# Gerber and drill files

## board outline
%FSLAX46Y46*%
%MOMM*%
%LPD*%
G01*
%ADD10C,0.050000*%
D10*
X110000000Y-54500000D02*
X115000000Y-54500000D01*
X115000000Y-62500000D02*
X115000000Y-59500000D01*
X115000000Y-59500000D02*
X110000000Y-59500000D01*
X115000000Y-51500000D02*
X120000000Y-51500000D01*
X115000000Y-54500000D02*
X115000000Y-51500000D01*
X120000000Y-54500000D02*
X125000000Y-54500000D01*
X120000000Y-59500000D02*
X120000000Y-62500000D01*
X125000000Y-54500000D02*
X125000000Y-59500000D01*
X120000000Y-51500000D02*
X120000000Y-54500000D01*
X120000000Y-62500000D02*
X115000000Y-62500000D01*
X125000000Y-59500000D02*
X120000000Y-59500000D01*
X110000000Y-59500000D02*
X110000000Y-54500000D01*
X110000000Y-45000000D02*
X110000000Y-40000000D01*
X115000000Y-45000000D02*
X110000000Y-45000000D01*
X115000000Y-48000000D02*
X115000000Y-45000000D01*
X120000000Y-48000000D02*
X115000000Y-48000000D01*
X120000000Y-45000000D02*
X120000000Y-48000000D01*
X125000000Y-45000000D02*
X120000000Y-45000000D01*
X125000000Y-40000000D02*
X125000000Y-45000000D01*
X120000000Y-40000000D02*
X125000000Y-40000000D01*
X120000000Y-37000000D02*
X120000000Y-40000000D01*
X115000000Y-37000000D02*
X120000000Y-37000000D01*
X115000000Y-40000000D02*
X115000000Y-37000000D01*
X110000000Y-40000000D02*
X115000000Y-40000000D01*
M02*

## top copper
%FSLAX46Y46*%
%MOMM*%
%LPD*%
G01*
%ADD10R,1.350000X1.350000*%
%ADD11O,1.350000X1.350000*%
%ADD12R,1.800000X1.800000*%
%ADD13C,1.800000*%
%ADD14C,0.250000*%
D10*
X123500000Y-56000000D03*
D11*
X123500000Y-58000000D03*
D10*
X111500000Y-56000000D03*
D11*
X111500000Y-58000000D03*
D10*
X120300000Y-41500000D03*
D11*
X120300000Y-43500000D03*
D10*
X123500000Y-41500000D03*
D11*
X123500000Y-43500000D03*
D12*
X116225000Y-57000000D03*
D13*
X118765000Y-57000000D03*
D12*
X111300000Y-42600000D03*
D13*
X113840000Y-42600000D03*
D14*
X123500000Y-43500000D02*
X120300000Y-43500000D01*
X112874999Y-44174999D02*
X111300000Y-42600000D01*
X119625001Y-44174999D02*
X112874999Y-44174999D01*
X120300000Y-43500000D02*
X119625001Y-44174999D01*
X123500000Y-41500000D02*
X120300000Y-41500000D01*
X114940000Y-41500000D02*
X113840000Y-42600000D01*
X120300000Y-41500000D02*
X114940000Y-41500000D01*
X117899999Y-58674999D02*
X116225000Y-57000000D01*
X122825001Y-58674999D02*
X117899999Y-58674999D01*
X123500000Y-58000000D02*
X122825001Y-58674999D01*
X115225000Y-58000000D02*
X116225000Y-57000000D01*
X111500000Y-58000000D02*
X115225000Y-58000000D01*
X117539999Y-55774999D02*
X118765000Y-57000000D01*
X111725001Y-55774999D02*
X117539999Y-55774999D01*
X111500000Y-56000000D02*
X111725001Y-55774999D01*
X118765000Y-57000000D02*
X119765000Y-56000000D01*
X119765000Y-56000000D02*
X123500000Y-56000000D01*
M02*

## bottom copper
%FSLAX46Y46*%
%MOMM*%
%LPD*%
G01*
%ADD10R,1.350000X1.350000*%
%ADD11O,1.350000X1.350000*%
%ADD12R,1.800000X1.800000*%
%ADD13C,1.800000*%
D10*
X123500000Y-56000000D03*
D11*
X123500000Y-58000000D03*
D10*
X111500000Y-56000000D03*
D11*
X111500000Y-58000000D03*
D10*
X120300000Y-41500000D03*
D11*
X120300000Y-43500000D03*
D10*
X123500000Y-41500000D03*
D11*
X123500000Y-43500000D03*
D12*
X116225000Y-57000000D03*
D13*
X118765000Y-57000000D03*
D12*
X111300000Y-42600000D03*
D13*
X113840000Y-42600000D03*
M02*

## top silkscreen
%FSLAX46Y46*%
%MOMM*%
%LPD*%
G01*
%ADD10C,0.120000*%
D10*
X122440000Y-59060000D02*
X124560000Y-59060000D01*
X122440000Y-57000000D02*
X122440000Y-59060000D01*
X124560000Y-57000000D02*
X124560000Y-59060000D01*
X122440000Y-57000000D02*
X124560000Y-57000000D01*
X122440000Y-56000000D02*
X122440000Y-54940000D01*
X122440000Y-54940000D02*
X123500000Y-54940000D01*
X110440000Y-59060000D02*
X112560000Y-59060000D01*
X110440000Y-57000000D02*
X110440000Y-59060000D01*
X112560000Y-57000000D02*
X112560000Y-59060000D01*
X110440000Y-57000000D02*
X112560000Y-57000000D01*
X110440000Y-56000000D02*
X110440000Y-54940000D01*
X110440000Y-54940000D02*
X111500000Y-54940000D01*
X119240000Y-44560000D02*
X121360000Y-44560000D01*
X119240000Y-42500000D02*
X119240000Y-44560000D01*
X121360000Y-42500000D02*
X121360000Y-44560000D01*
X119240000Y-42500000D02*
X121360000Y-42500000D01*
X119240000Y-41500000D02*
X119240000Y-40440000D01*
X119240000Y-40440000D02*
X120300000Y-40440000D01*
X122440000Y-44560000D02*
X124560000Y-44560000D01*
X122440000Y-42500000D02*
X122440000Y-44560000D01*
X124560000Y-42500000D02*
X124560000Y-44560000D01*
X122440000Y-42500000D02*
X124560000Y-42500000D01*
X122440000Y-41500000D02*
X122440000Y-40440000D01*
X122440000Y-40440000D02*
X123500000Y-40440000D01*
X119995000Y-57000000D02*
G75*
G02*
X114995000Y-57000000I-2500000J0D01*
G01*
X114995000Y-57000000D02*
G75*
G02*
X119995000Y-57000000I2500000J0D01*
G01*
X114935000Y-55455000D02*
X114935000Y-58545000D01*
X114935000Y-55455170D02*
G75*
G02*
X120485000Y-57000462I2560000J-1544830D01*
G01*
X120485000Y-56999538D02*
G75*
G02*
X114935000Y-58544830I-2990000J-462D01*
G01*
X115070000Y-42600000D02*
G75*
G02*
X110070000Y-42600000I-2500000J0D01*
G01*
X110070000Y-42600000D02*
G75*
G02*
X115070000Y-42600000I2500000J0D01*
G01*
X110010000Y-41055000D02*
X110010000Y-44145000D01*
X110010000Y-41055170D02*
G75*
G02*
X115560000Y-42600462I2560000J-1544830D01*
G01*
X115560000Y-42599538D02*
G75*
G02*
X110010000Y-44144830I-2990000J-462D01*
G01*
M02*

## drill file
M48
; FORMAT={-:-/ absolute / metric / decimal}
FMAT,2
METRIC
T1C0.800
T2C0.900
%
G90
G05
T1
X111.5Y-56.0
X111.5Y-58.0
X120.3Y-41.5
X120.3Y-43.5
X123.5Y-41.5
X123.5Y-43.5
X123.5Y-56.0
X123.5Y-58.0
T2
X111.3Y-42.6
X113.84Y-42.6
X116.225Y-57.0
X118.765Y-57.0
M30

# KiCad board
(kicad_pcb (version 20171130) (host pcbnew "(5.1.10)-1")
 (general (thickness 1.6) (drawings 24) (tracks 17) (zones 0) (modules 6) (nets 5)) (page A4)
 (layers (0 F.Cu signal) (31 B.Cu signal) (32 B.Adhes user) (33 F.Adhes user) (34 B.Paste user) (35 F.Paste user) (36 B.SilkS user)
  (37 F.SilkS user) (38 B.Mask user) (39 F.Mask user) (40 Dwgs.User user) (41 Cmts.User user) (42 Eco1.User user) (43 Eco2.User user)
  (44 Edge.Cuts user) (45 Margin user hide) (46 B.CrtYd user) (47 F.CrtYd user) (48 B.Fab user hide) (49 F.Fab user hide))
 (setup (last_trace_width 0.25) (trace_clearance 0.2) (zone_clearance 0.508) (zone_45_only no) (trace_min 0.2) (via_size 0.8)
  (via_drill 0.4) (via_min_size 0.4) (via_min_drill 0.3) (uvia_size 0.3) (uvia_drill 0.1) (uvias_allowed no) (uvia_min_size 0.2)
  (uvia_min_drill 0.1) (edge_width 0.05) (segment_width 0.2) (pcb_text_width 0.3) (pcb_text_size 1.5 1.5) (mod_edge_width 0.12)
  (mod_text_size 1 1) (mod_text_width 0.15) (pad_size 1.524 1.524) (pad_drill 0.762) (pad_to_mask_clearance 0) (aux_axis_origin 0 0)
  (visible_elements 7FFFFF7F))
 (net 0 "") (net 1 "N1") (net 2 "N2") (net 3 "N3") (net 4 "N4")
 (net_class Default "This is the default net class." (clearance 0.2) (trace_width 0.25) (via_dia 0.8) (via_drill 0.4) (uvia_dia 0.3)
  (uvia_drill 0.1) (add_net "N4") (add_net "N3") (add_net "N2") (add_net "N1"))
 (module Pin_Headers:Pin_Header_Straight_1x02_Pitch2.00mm (layer F.Cu) (at 123.5 56)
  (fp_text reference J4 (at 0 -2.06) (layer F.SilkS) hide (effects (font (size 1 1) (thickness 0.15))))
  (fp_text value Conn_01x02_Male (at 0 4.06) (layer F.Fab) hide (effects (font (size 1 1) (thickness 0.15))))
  (fp_line (start -1.06 3.06) (end 1.06 3.06) (layer F.SilkS) (width 0.12))
  (fp_line (start -1.06 1) (end -1.06 3.06) (layer F.SilkS) (width 0.12))
  (fp_line (start 1.06 1) (end 1.06 3.06) (layer F.SilkS) (width 0.12))
  (fp_line (start -1.06 1) (end 1.06 1) (layer F.SilkS) (width 0.12))
  (fp_line (start -1.06 0) (end -1.06 -1.06) (layer F.SilkS) (width 0.12))
  (fp_line (start -1.06 -1.06) (end 0 -1.06) (layer F.SilkS) (width 0.12))
  (pad 1 thru_hole rect (at 0 0) (size 1.35 1.35) (drill 0.8) (layers *.Cu *.Mask) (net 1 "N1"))
  (pad 2 thru_hole oval (at 0 2) (size 1.35 1.35) (drill 0.8) (layers *.Cu *.Mask) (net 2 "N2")))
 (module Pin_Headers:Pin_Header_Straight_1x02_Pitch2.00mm (layer F.Cu) (at 111.5 56)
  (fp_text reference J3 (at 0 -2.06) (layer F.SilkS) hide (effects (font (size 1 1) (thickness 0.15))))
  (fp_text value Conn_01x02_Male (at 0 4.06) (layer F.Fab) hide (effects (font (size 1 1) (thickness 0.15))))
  (fp_line (start -1.06 3.06) (end 1.06 3.06) (layer F.SilkS) (width 0.12))
  (fp_line (start -1.06 1) (end -1.06 3.06) (layer F.SilkS) (width 0.12))
  (fp_line (start 1.06 1) (end 1.06 3.06) (layer F.SilkS) (width 0.12))
  (fp_line (start -1.06 1) (end 1.06 1) (layer F.SilkS) (width 0.12))
  (fp_line (start -1.06 0) (end -1.06 -1.06) (layer F.SilkS) (width 0.12))
  (fp_line (start -1.06 -1.06) (end 0 -1.06) (layer F.SilkS) (width 0.12))
  (pad 1 thru_hole rect (at 0 0) (size 1.35 1.35) (drill 0.8) (layers *.Cu *.Mask) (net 1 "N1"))
  (pad 2 thru_hole oval (at 0 2) (size 1.35 1.35) (drill 0.8) (layers *.Cu *.Mask) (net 2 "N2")))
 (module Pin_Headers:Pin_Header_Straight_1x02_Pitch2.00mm (layer F.Cu) (at 120.3 41.5)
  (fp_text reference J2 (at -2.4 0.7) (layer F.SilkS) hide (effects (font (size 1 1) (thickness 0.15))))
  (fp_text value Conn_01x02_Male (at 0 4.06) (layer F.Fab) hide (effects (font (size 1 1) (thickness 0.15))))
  (fp_line (start -1.06 3.06) (end 1.06 3.06) (layer F.SilkS) (width 0.12))
  (fp_line (start -1.06 1) (end -1.06 3.06) (layer F.SilkS) (width 0.12))
  (fp_line (start 1.06 1) (end 1.06 3.06) (layer F.SilkS) (width 0.12))
  (fp_line (start -1.06 1) (end 1.06 1) (layer F.SilkS) (width 0.12))
  (fp_line (start -1.06 0) (end -1.06 -1.06) (layer F.SilkS) (width 0.12))
  (fp_line (start -1.06 -1.06) (end 0 -1.06) (layer F.SilkS) (width 0.12))
  (pad 1 thru_hole rect (at 0 0) (size 1.35 1.35) (drill 0.8) (layers *.Cu *.Mask) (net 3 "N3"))
  (pad 2 thru_hole oval (at 0 2) (size 1.35 1.35) (drill 0.8) (layers *.Cu *.Mask) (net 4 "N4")))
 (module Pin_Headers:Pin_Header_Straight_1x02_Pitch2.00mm (layer F.Cu) (at 123.5 41.5)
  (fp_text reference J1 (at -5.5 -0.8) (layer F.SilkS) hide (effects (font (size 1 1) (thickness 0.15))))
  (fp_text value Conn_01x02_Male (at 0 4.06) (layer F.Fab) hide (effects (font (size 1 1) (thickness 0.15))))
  (fp_line (start -1.06 3.06) (end 1.06 3.06) (layer F.SilkS) (width 0.12))
  (fp_line (start -1.06 1) (end -1.06 3.06) (layer F.SilkS) (width 0.12))
  (fp_line (start 1.06 1) (end 1.06 3.06) (layer F.SilkS) (width 0.12))
  (fp_line (start -1.06 1) (end 1.06 1) (layer F.SilkS) (width 0.12))
  (fp_line (start -1.06 0) (end -1.06 -1.06) (layer F.SilkS) (width 0.12))
  (fp_line (start -1.06 -1.06) (end 0 -1.06) (layer F.SilkS) (width 0.12))
  (pad 1 thru_hole rect (at 0 0) (size 1.35 1.35) (drill 0.8) (layers *.Cu *.Mask) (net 3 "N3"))
  (pad 2 thru_hole oval (at 0 2) (size 1.35 1.35) (drill 0.8) (layers *.Cu *.Mask) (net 4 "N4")))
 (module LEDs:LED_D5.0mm (layer F.Cu) (at 116.225 57)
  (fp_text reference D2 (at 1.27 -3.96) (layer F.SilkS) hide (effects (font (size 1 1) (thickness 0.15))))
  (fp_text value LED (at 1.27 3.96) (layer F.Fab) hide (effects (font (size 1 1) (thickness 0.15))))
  (fp_circle (center 1.27 0) (end 3.77 0) (layer F.SilkS) (width 0.12))
  (fp_line (start -1.29 -1.545) (end -1.29 1.545) (layer F.SilkS) (width 0.12))
  (fp_arc (start 1.27 0) (end -1.29 -1.54483) (angle 148.9) (layer F.SilkS) (width 0.12))
  (fp_arc (start 1.27 0) (end -1.29 1.54483) (angle -148.9) (layer F.SilkS) (width 0.12))
  (pad 1 thru_hole rect (at 0 0) (size 1.8 1.8) (drill 0.9) (layers *.Cu *.Mask) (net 2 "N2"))
  (pad 2 thru_hole circle (at 2.54 0) (size 1.8 1.8) (drill 0.9) (layers *.Cu *.Mask) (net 1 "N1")))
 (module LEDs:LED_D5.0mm (layer F.Cu) (at 111.3 42.6)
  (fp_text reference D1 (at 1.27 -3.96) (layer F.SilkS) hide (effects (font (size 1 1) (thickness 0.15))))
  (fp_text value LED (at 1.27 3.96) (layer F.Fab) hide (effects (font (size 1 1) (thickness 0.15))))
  (fp_circle (center 1.27 0) (end 3.77 0) (layer F.SilkS) (width 0.12))
  (fp_line (start -1.29 -1.545) (end -1.29 1.545) (layer F.SilkS) (width 0.12))
  (fp_arc (start 1.27 0) (end -1.29 -1.54483) (angle 148.9) (layer F.SilkS) (width 0.12))
  (fp_arc (start 1.27 0) (end -1.29 1.54483) (angle -148.9) (layer F.SilkS) (width 0.12))
  (pad 1 thru_hole rect (at 0 0) (size 1.8 1.8) (drill 0.9) (layers *.Cu *.Mask) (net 4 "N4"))
  (pad 2 thru_hole circle (at 2.54 0) (size 1.8 1.8) (drill 0.9) (layers *.Cu *.Mask) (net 3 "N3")))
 (gr_line (start 110 54.5) (end 115 54.5) (layer Edge.Cuts) (width 0.05))
 (gr_line (start 115 62.5) (end 115 59.5) (layer Edge.Cuts) (width 0.05))
 (gr_line (start 115 59.5) (end 110 59.5) (layer Edge.Cuts) (width 0.05))
 (gr_line (start 115 51.5) (end 120 51.5) (layer Edge.Cuts) (width 0.05))
 (gr_line (start 115 54.5) (end 115 51.5) (layer Edge.Cuts) (width 0.05))
 (gr_line (start 120 54.5) (end 125 54.5) (layer Edge.Cuts) (width 0.05))
 (gr_line (start 120 59.5) (end 120 62.5) (layer Edge.Cuts) (width 0.05))
 (gr_line (start 125 54.5) (end 125 59.5) (layer Edge.Cuts) (width 0.05))
 (gr_line (start 120 51.5) (end 120 54.5) (layer Edge.Cuts) (width 0.05))
 (gr_line (start 120 62.5) (end 115 62.5) (layer Edge.Cuts) (width 0.05))
 (gr_line (start 125 59.5) (end 120 59.5) (layer Edge.Cuts) (width 0.05))
 (gr_line (start 110 59.5) (end 110 54.5) (layer Edge.Cuts) (width 0.05))
 (gr_line (start 110 45) (end 110 40) (layer Edge.Cuts) (width 0.05))
 (gr_line (start 115 45) (end 110 45) (layer Edge.Cuts) (width 0.05))
 (gr_line (start 115 48) (end 115 45) (layer Edge.Cuts) (width 0.05))
 (gr_line (start 120 48) (end 115 48) (layer Edge.Cuts) (width 0.05))
 (gr_line (start 120 45) (end 120 48) (layer Edge.Cuts) (width 0.05))
 (gr_line (start 125 45) (end 120 45) (layer Edge.Cuts) (width 0.05))
 (gr_line (start 125 40) (end 125 45) (layer Edge.Cuts) (width 0.05))
 (gr_line (start 120 40) (end 125 40) (layer Edge.Cuts) (width 0.05))
 (gr_line (start 120 37) (end 120 40) (layer Edge.Cuts) (width 0.05))
 (gr_line (start 115 37) (end 120 37) (layer Edge.Cuts) (width 0.05))
 (gr_line (start 115 40) (end 115 37) (layer Edge.Cuts) (width 0.05))
 (gr_line (start 110 40) (end 115 40) (layer Edge.Cuts) (width 0.05))
 (segment (start 123.5 43.5) (end 120.3 43.5) (width 0.25) (layer F.Cu) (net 4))
 (segment (start 112.874999 44.174999) (end 111.3 42.6) (width 0.25) (layer F.Cu) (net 4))
 (segment (start 119.625001 44.174999) (end 112.874999 44.174999) (width 0.25) (layer F.Cu) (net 4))
 (segment (start 120.3 43.5) (end 119.625001 44.174999) (width 0.25) (layer F.Cu) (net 4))
 (segment (start 123.5 41.5) (end 120.3 41.5) (width 0.25) (layer F.Cu) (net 3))
 (segment (start 114.94 41.5) (end 113.84 42.6) (width 0.25) (layer F.Cu) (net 3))
 (segment (start 120.3 41.5) (end 114.94 41.5) (width 0.25) (layer F.Cu) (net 3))
 (segment (start 117.899999 58.674999) (end 116.225 57) (width 0.25) (layer F.Cu) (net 2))
 (segment (start 122.825001 58.674999) (end 117.899999 58.674999) (width 0.25) (layer F.Cu) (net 2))
 (segment (start 123.5 58) (end 122.825001 58.674999) (width 0.25) (layer F.Cu) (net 2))
 (segment (start 115.225 58) (end 116.225 57) (width 0.25) (layer F.Cu) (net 2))
 (segment (start 111.5 58) (end 115.225 58) (width 0.25) (layer F.Cu) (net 2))
 (segment (start 117.539999 55.774999) (end 118.765 57) (width 0.25) (layer F.Cu) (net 1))
 (segment (start 111.725001 55.774999) (end 117.539999 55.774999) (width 0.25) (layer F.Cu) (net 1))
 (segment (start 111.5 56) (end 111.725001 55.774999) (width 0.25) (layer F.Cu) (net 1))
 (segment (start 118.765 57) (end 119.765 56) (width 0.25) (layer F.Cu) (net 1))
 (segment (start 119.765 56) (end 123.5 56) (width 0.25) (layer F.Cu) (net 1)))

